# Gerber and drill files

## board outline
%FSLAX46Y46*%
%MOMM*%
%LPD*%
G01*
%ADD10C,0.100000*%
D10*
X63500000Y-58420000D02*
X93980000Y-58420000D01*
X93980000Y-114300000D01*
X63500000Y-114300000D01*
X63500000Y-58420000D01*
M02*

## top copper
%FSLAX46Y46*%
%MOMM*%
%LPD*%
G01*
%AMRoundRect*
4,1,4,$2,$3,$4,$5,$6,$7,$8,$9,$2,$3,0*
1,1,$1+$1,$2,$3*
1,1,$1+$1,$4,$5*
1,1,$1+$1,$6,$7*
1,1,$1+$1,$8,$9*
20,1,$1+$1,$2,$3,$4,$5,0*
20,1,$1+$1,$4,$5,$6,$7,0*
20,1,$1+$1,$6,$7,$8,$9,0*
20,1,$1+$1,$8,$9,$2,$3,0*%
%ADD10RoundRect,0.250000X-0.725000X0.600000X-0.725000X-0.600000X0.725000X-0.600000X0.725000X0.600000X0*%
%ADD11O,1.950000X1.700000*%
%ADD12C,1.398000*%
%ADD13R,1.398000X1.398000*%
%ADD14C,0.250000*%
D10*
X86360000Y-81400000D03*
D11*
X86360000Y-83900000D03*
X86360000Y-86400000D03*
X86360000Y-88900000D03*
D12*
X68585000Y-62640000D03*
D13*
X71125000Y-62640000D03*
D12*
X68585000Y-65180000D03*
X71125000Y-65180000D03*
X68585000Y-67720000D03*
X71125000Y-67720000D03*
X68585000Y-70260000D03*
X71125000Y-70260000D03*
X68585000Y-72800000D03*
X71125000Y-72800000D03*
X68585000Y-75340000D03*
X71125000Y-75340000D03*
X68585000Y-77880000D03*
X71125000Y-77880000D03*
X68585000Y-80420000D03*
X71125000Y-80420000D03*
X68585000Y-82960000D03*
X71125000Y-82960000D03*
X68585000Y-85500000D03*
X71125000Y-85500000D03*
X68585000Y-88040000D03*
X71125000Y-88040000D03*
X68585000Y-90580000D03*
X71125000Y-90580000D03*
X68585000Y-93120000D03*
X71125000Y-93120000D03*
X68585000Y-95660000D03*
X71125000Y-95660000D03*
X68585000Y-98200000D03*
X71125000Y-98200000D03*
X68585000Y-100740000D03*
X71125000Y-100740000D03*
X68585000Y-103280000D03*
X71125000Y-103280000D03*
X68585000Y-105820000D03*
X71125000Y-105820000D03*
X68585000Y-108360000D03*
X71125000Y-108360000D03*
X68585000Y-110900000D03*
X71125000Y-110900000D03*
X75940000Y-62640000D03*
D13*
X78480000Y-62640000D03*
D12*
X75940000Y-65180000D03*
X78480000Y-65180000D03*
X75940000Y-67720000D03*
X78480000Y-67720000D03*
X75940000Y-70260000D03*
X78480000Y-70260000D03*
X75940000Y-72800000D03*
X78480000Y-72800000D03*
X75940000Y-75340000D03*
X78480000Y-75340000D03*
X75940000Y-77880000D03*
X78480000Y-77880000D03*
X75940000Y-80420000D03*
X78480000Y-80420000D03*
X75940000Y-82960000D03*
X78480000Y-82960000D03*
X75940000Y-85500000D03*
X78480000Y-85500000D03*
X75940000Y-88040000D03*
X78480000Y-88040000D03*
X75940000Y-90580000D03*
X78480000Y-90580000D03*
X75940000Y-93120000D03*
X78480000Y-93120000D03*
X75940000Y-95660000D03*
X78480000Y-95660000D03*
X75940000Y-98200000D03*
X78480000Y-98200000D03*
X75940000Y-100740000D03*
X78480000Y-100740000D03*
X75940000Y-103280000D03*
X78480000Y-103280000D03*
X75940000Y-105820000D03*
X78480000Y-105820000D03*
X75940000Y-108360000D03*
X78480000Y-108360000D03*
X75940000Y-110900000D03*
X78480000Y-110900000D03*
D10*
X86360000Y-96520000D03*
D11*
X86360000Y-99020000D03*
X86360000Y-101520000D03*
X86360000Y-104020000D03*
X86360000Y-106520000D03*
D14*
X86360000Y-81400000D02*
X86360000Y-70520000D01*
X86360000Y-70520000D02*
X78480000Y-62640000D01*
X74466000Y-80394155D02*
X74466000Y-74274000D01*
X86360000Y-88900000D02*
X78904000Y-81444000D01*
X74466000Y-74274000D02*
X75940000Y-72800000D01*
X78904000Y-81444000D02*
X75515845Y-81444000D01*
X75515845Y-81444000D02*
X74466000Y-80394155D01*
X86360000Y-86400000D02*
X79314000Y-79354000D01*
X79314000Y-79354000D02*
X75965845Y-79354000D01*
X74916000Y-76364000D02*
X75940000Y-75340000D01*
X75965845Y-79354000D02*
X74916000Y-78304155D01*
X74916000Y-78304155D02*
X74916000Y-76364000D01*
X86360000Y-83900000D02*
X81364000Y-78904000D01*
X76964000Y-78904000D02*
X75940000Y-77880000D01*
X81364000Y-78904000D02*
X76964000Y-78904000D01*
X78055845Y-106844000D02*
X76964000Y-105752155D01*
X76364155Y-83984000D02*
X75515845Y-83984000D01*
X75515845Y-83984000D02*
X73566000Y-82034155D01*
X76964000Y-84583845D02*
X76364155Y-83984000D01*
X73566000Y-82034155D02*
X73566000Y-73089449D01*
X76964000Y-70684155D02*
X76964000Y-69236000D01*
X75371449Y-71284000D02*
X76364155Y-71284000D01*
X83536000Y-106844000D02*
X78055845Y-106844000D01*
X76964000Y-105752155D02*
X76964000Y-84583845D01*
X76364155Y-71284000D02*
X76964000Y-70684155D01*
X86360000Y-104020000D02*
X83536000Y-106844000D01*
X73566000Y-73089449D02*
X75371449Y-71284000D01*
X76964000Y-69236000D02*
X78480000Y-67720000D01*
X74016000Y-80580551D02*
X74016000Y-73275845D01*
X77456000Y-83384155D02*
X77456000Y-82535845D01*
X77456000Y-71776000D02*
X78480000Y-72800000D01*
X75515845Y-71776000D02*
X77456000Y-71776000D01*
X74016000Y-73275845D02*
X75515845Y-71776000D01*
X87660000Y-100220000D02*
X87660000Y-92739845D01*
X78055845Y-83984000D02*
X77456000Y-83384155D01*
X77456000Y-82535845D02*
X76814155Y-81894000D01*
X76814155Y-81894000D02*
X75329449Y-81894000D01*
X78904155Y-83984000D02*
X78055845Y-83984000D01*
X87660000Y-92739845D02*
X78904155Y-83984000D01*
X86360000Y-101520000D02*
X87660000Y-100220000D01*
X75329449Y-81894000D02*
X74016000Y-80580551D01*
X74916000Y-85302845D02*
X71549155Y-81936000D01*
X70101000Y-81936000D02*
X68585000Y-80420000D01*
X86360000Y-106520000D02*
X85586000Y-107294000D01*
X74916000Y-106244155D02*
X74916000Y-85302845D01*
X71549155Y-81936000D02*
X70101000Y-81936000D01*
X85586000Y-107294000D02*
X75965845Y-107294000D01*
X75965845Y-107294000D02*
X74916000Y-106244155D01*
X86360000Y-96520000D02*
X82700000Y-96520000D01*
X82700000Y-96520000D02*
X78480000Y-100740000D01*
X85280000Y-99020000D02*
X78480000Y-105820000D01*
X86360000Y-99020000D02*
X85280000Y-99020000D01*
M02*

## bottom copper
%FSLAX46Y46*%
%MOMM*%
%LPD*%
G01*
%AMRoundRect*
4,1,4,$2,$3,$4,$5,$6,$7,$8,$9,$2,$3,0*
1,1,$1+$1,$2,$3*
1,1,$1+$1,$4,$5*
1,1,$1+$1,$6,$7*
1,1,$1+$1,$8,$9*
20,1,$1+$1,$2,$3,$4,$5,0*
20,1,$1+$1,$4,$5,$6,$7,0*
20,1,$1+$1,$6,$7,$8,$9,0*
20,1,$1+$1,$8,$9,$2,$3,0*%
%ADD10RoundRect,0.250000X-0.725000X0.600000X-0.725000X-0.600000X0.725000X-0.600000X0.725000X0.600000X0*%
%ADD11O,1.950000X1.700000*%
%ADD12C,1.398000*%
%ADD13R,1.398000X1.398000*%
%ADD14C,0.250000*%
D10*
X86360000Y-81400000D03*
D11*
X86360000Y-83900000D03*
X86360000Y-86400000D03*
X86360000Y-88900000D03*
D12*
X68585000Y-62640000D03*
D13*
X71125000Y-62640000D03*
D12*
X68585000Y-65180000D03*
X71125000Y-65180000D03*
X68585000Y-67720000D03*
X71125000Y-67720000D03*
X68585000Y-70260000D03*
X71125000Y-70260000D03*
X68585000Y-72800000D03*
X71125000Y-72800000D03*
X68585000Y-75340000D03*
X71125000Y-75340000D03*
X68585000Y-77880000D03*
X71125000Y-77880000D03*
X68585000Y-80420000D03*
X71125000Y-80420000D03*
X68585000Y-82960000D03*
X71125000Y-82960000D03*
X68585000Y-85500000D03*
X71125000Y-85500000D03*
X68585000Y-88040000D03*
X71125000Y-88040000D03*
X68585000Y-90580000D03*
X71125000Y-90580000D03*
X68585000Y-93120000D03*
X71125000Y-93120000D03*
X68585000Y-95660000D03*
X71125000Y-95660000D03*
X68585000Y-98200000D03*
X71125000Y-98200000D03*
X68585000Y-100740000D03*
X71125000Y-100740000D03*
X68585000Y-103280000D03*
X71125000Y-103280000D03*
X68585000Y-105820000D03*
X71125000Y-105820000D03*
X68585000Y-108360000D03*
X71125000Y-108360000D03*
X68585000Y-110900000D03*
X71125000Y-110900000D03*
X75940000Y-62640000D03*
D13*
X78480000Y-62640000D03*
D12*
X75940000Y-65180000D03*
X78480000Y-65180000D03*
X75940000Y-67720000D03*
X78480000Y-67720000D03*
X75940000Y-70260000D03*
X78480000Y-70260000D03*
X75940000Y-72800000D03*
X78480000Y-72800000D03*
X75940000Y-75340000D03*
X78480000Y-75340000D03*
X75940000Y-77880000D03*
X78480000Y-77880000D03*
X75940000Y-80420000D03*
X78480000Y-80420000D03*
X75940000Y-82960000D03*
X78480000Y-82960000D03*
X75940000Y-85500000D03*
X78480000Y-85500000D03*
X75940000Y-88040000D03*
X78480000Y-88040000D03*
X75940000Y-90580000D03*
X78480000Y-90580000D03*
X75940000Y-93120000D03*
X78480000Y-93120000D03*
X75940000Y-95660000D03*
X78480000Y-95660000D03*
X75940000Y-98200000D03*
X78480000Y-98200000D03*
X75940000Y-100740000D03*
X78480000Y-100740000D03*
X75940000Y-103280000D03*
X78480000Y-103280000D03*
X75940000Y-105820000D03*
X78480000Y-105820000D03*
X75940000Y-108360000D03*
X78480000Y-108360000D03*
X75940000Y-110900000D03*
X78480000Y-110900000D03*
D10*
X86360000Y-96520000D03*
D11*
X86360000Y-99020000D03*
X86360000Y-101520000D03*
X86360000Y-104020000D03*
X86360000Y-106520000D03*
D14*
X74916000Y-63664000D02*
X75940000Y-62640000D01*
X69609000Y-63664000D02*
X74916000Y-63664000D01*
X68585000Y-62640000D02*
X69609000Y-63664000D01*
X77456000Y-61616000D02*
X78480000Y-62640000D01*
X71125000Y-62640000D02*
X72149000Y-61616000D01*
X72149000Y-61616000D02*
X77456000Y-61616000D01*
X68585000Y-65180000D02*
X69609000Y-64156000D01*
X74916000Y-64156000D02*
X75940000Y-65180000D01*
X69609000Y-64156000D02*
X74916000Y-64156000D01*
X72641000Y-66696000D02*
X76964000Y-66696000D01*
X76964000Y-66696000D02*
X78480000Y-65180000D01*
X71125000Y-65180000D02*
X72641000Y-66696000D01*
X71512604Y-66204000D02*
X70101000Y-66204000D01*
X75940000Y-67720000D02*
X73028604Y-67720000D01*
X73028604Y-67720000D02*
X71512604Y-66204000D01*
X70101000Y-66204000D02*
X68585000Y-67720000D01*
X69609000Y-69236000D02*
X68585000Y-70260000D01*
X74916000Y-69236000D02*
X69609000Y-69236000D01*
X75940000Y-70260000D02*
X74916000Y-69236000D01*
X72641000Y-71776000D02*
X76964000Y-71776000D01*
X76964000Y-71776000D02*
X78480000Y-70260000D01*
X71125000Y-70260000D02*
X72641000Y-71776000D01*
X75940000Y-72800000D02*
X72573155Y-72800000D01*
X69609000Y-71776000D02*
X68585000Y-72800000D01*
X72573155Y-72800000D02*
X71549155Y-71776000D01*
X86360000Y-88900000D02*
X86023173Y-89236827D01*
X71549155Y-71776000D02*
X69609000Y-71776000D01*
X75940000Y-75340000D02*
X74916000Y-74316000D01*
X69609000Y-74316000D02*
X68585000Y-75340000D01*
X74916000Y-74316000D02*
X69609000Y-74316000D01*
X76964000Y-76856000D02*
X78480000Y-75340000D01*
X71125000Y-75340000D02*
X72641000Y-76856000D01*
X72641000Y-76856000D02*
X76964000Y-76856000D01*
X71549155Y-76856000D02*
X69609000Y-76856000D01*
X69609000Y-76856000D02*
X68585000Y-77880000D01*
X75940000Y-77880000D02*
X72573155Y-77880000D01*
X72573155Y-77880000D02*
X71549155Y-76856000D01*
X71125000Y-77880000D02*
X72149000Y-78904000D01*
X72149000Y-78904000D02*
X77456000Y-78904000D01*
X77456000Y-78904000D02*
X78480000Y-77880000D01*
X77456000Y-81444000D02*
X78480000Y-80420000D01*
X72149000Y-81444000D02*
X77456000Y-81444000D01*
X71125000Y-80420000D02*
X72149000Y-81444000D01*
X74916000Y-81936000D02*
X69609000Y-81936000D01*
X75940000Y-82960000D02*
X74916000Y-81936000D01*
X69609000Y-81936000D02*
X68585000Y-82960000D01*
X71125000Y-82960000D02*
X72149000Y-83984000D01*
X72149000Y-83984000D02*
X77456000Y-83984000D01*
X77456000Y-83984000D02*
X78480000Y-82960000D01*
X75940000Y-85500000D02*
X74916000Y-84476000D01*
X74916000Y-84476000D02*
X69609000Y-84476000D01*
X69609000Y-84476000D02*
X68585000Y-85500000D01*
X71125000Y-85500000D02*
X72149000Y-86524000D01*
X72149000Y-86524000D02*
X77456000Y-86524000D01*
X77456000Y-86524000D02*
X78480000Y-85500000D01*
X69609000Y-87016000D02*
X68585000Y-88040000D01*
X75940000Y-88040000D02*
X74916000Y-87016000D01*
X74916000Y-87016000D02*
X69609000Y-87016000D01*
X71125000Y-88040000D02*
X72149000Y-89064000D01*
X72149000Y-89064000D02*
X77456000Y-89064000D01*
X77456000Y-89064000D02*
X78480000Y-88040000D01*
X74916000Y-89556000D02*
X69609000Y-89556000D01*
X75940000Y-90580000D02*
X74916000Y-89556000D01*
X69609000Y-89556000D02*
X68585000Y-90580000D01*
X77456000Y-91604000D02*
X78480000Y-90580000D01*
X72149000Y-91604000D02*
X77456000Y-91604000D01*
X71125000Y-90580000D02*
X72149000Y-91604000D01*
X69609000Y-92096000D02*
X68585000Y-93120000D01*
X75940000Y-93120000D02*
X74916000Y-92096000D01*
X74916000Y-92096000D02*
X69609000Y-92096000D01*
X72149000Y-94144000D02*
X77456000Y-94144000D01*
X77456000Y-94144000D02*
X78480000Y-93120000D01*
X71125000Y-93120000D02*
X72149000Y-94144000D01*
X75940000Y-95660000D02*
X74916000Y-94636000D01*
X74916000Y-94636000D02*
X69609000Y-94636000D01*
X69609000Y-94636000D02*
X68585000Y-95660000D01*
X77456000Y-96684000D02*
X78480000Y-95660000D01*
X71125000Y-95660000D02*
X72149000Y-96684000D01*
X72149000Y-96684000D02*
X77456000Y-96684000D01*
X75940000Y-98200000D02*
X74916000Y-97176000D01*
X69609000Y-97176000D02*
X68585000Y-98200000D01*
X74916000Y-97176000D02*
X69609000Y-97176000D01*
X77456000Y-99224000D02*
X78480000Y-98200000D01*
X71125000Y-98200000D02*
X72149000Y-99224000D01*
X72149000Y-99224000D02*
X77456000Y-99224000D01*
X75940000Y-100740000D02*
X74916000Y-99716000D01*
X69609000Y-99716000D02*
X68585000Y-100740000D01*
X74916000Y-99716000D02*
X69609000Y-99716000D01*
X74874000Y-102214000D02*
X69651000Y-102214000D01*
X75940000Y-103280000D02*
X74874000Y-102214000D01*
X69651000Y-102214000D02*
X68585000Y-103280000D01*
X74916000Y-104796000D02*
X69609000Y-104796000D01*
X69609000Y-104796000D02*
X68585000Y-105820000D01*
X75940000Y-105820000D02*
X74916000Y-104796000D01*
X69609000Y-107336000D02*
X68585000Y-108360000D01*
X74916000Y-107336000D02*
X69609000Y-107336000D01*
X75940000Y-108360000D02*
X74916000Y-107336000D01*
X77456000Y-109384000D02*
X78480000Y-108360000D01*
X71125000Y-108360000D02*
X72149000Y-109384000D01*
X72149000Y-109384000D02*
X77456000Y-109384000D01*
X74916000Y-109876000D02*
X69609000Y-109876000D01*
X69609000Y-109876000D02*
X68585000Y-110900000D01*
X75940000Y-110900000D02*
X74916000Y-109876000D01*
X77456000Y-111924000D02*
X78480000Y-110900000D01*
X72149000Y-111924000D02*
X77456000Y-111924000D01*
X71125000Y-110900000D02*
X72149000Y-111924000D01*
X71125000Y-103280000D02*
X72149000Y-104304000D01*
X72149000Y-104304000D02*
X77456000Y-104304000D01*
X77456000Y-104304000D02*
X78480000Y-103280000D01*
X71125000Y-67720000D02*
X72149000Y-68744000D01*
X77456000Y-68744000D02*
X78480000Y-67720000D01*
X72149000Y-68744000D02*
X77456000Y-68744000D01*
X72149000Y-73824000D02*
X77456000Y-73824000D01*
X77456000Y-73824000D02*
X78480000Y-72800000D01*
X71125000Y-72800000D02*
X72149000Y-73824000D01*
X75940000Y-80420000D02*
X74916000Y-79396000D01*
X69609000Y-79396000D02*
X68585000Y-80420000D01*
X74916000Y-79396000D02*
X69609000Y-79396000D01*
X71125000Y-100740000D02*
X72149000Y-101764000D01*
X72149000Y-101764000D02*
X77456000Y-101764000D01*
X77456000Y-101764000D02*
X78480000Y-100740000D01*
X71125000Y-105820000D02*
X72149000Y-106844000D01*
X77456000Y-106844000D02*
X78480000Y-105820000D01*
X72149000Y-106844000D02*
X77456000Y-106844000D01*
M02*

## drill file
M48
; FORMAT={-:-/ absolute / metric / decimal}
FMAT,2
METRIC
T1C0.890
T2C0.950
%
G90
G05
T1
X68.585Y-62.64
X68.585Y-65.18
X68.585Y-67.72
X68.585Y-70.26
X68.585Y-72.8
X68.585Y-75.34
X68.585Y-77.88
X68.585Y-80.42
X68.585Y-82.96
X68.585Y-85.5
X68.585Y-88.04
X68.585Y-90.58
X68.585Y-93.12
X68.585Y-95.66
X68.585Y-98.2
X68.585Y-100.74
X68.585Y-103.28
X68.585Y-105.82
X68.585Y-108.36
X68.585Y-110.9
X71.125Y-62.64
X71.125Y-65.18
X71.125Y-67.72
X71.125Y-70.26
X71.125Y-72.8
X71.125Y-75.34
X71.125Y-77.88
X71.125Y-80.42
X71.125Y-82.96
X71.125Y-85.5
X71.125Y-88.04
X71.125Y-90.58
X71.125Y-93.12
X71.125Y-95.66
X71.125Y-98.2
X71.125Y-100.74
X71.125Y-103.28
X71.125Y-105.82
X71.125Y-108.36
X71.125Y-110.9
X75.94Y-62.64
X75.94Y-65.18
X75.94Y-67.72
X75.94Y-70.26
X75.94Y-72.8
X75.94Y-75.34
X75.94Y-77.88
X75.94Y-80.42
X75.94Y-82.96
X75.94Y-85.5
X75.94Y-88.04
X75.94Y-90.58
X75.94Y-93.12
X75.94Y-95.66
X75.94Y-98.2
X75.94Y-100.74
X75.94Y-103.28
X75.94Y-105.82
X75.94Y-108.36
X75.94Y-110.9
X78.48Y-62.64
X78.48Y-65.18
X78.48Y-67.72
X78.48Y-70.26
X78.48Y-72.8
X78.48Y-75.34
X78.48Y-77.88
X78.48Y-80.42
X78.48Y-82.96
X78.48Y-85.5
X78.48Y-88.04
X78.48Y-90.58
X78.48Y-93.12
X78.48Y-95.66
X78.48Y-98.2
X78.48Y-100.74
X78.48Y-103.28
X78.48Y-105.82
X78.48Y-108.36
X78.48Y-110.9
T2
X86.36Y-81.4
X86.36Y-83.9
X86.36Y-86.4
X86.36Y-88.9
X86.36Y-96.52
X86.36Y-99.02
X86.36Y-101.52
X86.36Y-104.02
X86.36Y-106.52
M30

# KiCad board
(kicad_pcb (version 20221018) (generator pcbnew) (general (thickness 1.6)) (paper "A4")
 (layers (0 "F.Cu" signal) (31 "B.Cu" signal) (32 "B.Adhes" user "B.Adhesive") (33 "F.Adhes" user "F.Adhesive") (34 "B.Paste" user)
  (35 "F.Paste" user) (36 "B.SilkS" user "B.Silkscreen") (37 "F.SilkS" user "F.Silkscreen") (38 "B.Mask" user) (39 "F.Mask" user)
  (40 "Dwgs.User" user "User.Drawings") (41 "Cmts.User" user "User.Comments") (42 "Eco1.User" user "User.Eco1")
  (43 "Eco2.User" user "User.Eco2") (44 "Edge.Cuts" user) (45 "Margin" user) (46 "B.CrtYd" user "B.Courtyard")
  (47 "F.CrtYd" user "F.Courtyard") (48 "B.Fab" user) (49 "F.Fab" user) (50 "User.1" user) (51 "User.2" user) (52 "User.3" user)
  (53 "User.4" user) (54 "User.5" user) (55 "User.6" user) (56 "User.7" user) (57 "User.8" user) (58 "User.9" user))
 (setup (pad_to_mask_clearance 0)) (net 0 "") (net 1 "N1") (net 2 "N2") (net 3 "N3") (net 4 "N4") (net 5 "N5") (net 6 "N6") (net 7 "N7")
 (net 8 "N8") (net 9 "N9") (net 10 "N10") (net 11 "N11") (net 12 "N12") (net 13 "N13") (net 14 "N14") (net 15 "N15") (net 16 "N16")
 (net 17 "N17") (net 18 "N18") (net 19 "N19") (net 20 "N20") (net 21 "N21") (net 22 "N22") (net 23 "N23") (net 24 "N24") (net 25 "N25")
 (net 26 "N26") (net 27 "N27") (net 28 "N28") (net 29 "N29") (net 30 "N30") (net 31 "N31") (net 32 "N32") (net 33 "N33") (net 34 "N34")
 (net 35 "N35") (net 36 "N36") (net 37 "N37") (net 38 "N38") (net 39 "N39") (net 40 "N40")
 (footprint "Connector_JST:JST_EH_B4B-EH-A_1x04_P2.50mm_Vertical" (layer "F.Cu") (at 86.36 81.4 -90)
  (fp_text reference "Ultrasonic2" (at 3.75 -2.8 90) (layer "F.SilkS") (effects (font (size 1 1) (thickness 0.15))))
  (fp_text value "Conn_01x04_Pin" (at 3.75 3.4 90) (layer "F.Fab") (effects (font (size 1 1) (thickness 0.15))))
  (pad "1" thru_hole roundrect (at 0 0 270) (size 1.7 1.95) (drill 0.95) (layers "*.Cu" "*.Mask") (roundrect_rratio 0.1470588235)
   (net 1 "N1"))
  (pad "2" thru_hole oval (at 2.5 0 270) (size 1.7 1.95) (drill 0.95) (layers "*.Cu" "*.Mask") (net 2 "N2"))
  (pad "3" thru_hole oval (at 5 0 270) (size 1.7 1.95) (drill 0.95) (layers "*.Cu" "*.Mask") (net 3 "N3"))
  (pad "4" thru_hole oval (at 7.5 0 270) (size 1.7 1.95) (drill 0.95) (layers "*.Cu" "*.Mask") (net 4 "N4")))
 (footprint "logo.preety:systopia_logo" (layer "F.Cu") (at 87.63 68.58)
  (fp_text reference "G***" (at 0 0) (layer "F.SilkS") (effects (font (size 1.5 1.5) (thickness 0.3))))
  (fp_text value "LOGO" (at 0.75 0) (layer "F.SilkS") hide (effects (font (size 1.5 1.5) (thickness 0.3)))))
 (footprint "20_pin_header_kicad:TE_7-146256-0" (layer "F.Cu") (at 69.855 86.77 -90)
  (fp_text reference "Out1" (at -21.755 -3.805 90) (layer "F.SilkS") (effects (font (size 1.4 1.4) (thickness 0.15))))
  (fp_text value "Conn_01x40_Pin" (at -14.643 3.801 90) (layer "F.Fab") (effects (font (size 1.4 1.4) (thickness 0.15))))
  (pad "1" thru_hole circle (at -24.13 1.27 270) (size 1.398 1.398) (drill 0.89) (layers "*.Cu" "*.Mask") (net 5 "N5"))
  (pad "2" thru_hole rect (at -24.13 -1.27 270) (size 1.398 1.398) (drill 0.89) (layers "*.Cu" "*.Mask") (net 1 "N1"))
  (pad "3" thru_hole circle (at -21.59 1.27 270) (size 1.398 1.398) (drill 0.89) (layers "*.Cu" "*.Mask") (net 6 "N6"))
  (pad "4" thru_hole circle (at -21.59 -1.27 270) (size 1.398 1.398) (drill 0.89) (layers "*.Cu" "*.Mask") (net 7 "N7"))
  (pad "5" thru_hole circle (at -19.05 1.27 270) (size 1.398 1.398) (drill 0.89) (layers "*.Cu" "*.Mask") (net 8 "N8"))
  (pad "6" thru_hole circle (at -19.05 -1.27 270) (size 1.398 1.398) (drill 0.89) (layers "*.Cu" "*.Mask") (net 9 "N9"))
  (pad "7" thru_hole circle (at -16.51 1.27 270) (size 1.398 1.398) (drill 0.89) (layers "*.Cu" "*.Mask") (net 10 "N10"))
  (pad "8" thru_hole circle (at -16.51 -1.27 270) (size 1.398 1.398) (drill 0.89) (layers "*.Cu" "*.Mask") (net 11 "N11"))
  (pad "9" thru_hole circle (at -13.97 1.27 270) (size 1.398 1.398) (drill 0.89) (layers "*.Cu" "*.Mask") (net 4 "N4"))
  (pad "10" thru_hole circle (at -13.97 -1.27 270) (size 1.398 1.398) (drill 0.89) (layers "*.Cu" "*.Mask") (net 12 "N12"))
  (pad "11" thru_hole circle (at -11.43 1.27 270) (size 1.398 1.398) (drill 0.89) (layers "*.Cu" "*.Mask") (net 3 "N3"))
  (pad "12" thru_hole circle (at -11.43 -1.27 270) (size 1.398 1.398) (drill 0.89) (layers "*.Cu" "*.Mask") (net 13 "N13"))
  (pad "13" thru_hole circle (at -8.89 1.27 270) (size 1.398 1.398) (drill 0.89) (layers "*.Cu" "*.Mask") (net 2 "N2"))
  (pad "14" thru_hole circle (at -8.89 -1.27 270) (size 1.398 1.398) (drill 0.89) (layers "*.Cu" "*.Mask") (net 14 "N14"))
  (pad "15" thru_hole circle (at -6.35 1.27 270) (size 1.398 1.398) (drill 0.89) (layers "*.Cu" "*.Mask") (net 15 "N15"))
  (pad "16" thru_hole circle (at -6.35 -1.27 270) (size 1.398 1.398) (drill 0.89) (layers "*.Cu" "*.Mask") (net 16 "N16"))
  (pad "17" thru_hole circle (at -3.81 1.27 270) (size 1.398 1.398) (drill 0.89) (layers "*.Cu" "*.Mask") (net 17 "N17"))
  (pad "18" thru_hole circle (at -3.81 -1.27 270) (size 1.398 1.398) (drill 0.89) (layers "*.Cu" "*.Mask") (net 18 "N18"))
  (pad "19" thru_hole circle (at -1.27 1.27 270) (size 1.398 1.398) (drill 0.89) (layers "*.Cu" "*.Mask") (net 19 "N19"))
  (pad "20" thru_hole circle (at -1.27 -1.27 270) (size 1.398 1.398) (drill 0.89) (layers "*.Cu" "*.Mask") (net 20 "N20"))
  (pad "21" thru_hole circle (at 1.27 1.27 270) (size 1.398 1.398) (drill 0.89) (layers "*.Cu" "*.Mask") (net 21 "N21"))
  (pad "22" thru_hole circle (at 1.27 -1.27 270) (size 1.398 1.398) (drill 0.89) (layers "*.Cu" "*.Mask") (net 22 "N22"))
  (pad "23" thru_hole circle (at 3.81 1.27 270) (size 1.398 1.398) (drill 0.89) (layers "*.Cu" "*.Mask") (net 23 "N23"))
  (pad "24" thru_hole circle (at 3.81 -1.27 270) (size 1.398 1.398) (drill 0.89) (layers "*.Cu" "*.Mask") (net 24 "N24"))
  (pad "25" thru_hole circle (at 6.35 1.27 270) (size 1.398 1.398) (drill 0.89) (layers "*.Cu" "*.Mask") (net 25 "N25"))
  (pad "26" thru_hole circle (at 6.35 -1.27 270) (size 1.398 1.398) (drill 0.89) (layers "*.Cu" "*.Mask") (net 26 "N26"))
  (pad "27" thru_hole circle (at 8.89 1.27 270) (size 1.398 1.398) (drill 0.89) (layers "*.Cu" "*.Mask") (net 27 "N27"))
  (pad "28" thru_hole circle (at 8.89 -1.27 270) (size 1.398 1.398) (drill 0.89) (layers "*.Cu" "*.Mask") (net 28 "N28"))
  (pad "29" thru_hole circle (at 11.43 1.27 270) (size 1.398 1.398) (drill 0.89) (layers "*.Cu" "*.Mask") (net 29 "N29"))
  (pad "30" thru_hole circle (at 11.43 -1.27 270) (size 1.398 1.398) (drill 0.89) (layers "*.Cu" "*.Mask") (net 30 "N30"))
  (pad "31" thru_hole circle (at 13.97 1.27 270) (size 1.398 1.398) (drill 0.89) (layers "*.Cu" "*.Mask") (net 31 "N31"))
  (pad "32" thru_hole circle (at 13.97 -1.27 270) (size 1.398 1.398) (drill 0.89) (layers "*.Cu" "*.Mask") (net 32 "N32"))
  (pad "33" thru_hole circle (at 16.51 1.27 270) (size 1.398 1.398) (drill 0.89) (layers "*.Cu" "*.Mask") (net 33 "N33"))
  (pad "34" thru_hole circle (at 16.51 -1.27 270) (size 1.398 1.398) (drill 0.89) (layers "*.Cu" "*.Mask") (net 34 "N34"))
  (pad "35" thru_hole circle (at 19.05 1.27 270) (size 1.398 1.398) (drill 0.89) (layers "*.Cu" "*.Mask") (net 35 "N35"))
  (pad "36" thru_hole circle (at 19.05 -1.27 270) (size 1.398 1.398) (drill 0.89) (layers "*.Cu" "*.Mask") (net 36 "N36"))
  (pad "37" thru_hole circle (at 21.59 1.27 270) (size 1.398 1.398) (drill 0.89) (layers "*.Cu" "*.Mask") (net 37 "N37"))
  (pad "38" thru_hole circle (at 21.59 -1.27 270) (size 1.398 1.398) (drill 0.89) (layers "*.Cu" "*.Mask") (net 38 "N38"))
  (pad "39" thru_hole circle (at 24.13 1.27 270) (size 1.398 1.398) (drill 0.89) (layers "*.Cu" "*.Mask") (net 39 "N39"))
  (pad "40" thru_hole circle (at 24.13 -1.27 270) (size 1.398 1.398) (drill 0.89) (layers "*.Cu" "*.Mask") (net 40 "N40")))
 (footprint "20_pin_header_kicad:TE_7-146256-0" (layer "F.Cu") (at 77.21 86.77 -90)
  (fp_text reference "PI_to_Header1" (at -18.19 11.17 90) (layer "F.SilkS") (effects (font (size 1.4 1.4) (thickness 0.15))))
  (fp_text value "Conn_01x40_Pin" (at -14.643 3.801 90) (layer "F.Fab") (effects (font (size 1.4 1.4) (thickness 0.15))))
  (pad "1" thru_hole circle (at -24.13 1.27 270) (size 1.398 1.398) (drill 0.89) (layers "*.Cu" "*.Mask") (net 5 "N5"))
  (pad "2" thru_hole rect (at -24.13 -1.27 270) (size 1.398 1.398) (drill 0.89) (layers "*.Cu" "*.Mask") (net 1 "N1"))
  (pad "3" thru_hole circle (at -21.59 1.27 270) (size 1.398 1.398) (drill 0.89) (layers "*.Cu" "*.Mask") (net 6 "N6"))
  (pad "4" thru_hole circle (at -21.59 -1.27 270) (size 1.398 1.398) (drill 0.89) (layers "*.Cu" "*.Mask") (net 7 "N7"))
  (pad "5" thru_hole circle (at -19.05 1.27 270) (size 1.398 1.398) (drill 0.89) (layers "*.Cu" "*.Mask") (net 8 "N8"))
  (pad "6" thru_hole circle (at -19.05 -1.27 270) (size 1.398 1.398) (drill 0.89) (layers "*.Cu" "*.Mask") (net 9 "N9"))
  (pad "7" thru_hole circle (at -16.51 1.27 270) (size 1.398 1.398) (drill 0.89) (layers "*.Cu" "*.Mask") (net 10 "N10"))
  (pad "8" thru_hole circle (at -16.51 -1.27 270) (size 1.398 1.398) (drill 0.89) (layers "*.Cu" "*.Mask") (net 11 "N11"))
  (pad "9" thru_hole circle (at -13.97 1.27 270) (size 1.398 1.398) (drill 0.89) (layers "*.Cu" "*.Mask") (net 4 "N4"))
  (pad "10" thru_hole circle (at -13.97 -1.27 270) (size 1.398 1.398) (drill 0.89) (layers "*.Cu" "*.Mask") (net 12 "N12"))
  (pad "11" thru_hole circle (at -11.43 1.27 270) (size 1.398 1.398) (drill 0.89) (layers "*.Cu" "*.Mask") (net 3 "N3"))
  (pad "12" thru_hole circle (at -11.43 -1.27 270) (size 1.398 1.398) (drill 0.89) (layers "*.Cu" "*.Mask") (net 13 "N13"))
  (pad "13" thru_hole circle (at -8.89 1.27 270) (size 1.398 1.398) (drill 0.89) (layers "*.Cu" "*.Mask") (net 2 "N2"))
  (pad "14" thru_hole circle (at -8.89 -1.27 270) (size 1.398 1.398) (drill 0.89) (layers "*.Cu" "*.Mask") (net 14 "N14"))
  (pad "15" thru_hole circle (at -6.35 1.27 270) (size 1.398 1.398) (drill 0.89) (layers "*.Cu" "*.Mask") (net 15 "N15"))
  (pad "16" thru_hole circle (at -6.35 -1.27 270) (size 1.398 1.398) (drill 0.89) (layers "*.Cu" "*.Mask") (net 16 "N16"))
  (pad "17" thru_hole circle (at -3.81 1.27 270) (size 1.398 1.398) (drill 0.89) (layers "*.Cu" "*.Mask") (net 17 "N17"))
  (pad "18" thru_hole circle (at -3.81 -1.27 270) (size 1.398 1.398) (drill 0.89) (layers "*.Cu" "*.Mask") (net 18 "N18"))
  (pad "19" thru_hole circle (at -1.27 1.27 270) (size 1.398 1.398) (drill 0.89) (layers "*.Cu" "*.Mask") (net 19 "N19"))
  (pad "20" thru_hole circle (at -1.27 -1.27 270) (size 1.398 1.398) (drill 0.89) (layers "*.Cu" "*.Mask") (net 20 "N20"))
  (pad "21" thru_hole circle (at 1.27 1.27 270) (size 1.398 1.398) (drill 0.89) (layers "*.Cu" "*.Mask") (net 21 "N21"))
  (pad "22" thru_hole circle (at 1.27 -1.27 270) (size 1.398 1.398) (drill 0.89) (layers "*.Cu" "*.Mask") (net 22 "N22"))
  (pad "23" thru_hole circle (at 3.81 1.27 270) (size 1.398 1.398) (drill 0.89) (layers "*.Cu" "*.Mask") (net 23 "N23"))
  (pad "24" thru_hole circle (at 3.81 -1.27 270) (size 1.398 1.398) (drill 0.89) (layers "*.Cu" "*.Mask") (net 24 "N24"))
  (pad "25" thru_hole circle (at 6.35 1.27 270) (size 1.398 1.398) (drill 0.89) (layers "*.Cu" "*.Mask") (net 25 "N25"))
  (pad "26" thru_hole circle (at 6.35 -1.27 270) (size 1.398 1.398) (drill 0.89) (layers "*.Cu" "*.Mask") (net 26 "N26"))
  (pad "27" thru_hole circle (at 8.89 1.27 270) (size 1.398 1.398) (drill 0.89) (layers "*.Cu" "*.Mask") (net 27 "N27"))
  (pad "28" thru_hole circle (at 8.89 -1.27 270) (size 1.398 1.398) (drill 0.89) (layers "*.Cu" "*.Mask") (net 28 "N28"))
  (pad "29" thru_hole circle (at 11.43 1.27 270) (size 1.398 1.398) (drill 0.89) (layers "*.Cu" "*.Mask") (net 29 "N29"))
  (pad "30" thru_hole circle (at 11.43 -1.27 270) (size 1.398 1.398) (drill 0.89) (layers "*.Cu" "*.Mask") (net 30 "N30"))
  (pad "31" thru_hole circle (at 13.97 1.27 270) (size 1.398 1.398) (drill 0.89) (layers "*.Cu" "*.Mask") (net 31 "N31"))
  (pad "32" thru_hole circle (at 13.97 -1.27 270) (size 1.398 1.398) (drill 0.89) (layers "*.Cu" "*.Mask") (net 32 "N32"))
  (pad "33" thru_hole circle (at 16.51 1.27 270) (size 1.398 1.398) (drill 0.89) (layers "*.Cu" "*.Mask") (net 33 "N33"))
  (pad "34" thru_hole circle (at 16.51 -1.27 270) (size 1.398 1.398) (drill 0.89) (layers "*.Cu" "*.Mask") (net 34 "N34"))
  (pad "35" thru_hole circle (at 19.05 1.27 270) (size 1.398 1.398) (drill 0.89) (layers "*.Cu" "*.Mask") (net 35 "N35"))
  (pad "36" thru_hole circle (at 19.05 -1.27 270) (size 1.398 1.398) (drill 0.89) (layers "*.Cu" "*.Mask") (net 36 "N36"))
  (pad "37" thru_hole circle (at 21.59 1.27 270) (size 1.398 1.398) (drill 0.89) (layers "*.Cu" "*.Mask") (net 37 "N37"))
  (pad "38" thru_hole circle (at 21.59 -1.27 270) (size 1.398 1.398) (drill 0.89) (layers "*.Cu" "*.Mask") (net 38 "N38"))
  (pad "39" thru_hole circle (at 24.13 1.27 270) (size 1.398 1.398) (drill 0.89) (layers "*.Cu" "*.Mask") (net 39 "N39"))
  (pad "40" thru_hole circle (at 24.13 -1.27 270) (size 1.398 1.398) (drill 0.89) (layers "*.Cu" "*.Mask") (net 40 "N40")))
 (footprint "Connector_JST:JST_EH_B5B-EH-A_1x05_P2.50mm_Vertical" (layer "F.Cu") (at 86.36 96.52 -90)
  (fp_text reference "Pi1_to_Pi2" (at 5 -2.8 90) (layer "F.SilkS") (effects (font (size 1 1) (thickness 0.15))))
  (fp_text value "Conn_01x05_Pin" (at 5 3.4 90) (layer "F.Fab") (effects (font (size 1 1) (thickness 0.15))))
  (pad "1" thru_hole roundrect (at 0 0 270) (size 1.7 1.95) (drill 0.95) (layers "*.Cu" "*.Mask") (roundrect_rratio 0.147059) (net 32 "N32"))
  (pad "2" thru_hole oval (at 2.5 0 270) (size 1.7 1.95) (drill 0.95) (layers "*.Cu" "*.Mask") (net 36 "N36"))
  (pad "3" thru_hole oval (at 5 0 270) (size 1.7 1.95) (drill 0.95) (layers "*.Cu" "*.Mask") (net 12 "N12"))
  (pad "4" thru_hole oval (at 7.5 0 270) (size 1.7 1.95) (drill 0.95) (layers "*.Cu" "*.Mask") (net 9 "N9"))
  (pad "5" thru_hole oval (at 10 0 270) (size 1.7 1.95) (drill 0.95) (layers "*.Cu" "*.Mask") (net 15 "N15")))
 (gr_rect (start 63.5 58.42) (end 93.98 114.3) (stroke (width 0.1) (type default)) (fill none) (layer "Edge.Cuts"))
 (segment (start 74.916 63.664) (end 75.94 62.64) (width 0.25) (layer "B.Cu") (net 5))
 (segment (start 69.609 63.664) (end 74.916 63.664) (width 0.25) (layer "B.Cu") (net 5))
 (segment (start 68.585 62.64) (end 69.609 63.664) (width 0.25) (layer "B.Cu") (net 5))
 (segment (start 86.36 81.4) (end 86.36 70.52) (width 0.25) (layer "F.Cu") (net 1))
 (segment (start 86.36 70.52) (end 78.48 62.64) (width 0.25) (layer "F.Cu") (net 1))
 (segment (start 77.456 61.616) (end 78.48 62.64) (width 0.25) (layer "B.Cu") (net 1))
 (segment (start 71.125 62.64) (end 72.149 61.616) (width 0.25) (layer "B.Cu") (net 1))
 (segment (start 72.149 61.616) (end 77.456 61.616) (width 0.25) (layer "B.Cu") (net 1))
 (segment (start 68.585 65.18) (end 69.609 64.156) (width 0.25) (layer "B.Cu") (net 6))
 (segment (start 74.916 64.156) (end 75.94 65.18) (width 0.25) (layer "B.Cu") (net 6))
 (segment (start 69.609 64.156) (end 74.916 64.156) (width 0.25) (layer "B.Cu") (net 6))
 (segment (start 72.641 66.696) (end 76.964 66.696) (width 0.25) (layer "B.Cu") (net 7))
 (segment (start 76.964 66.696) (end 78.48 65.18) (width 0.25) (layer "B.Cu") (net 7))
 (segment (start 71.125 65.18) (end 72.641 66.696) (width 0.25) (layer "B.Cu") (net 7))
 (segment (start 71.512604 66.204) (end 70.101 66.204) (width 0.25) (layer "B.Cu") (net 8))
 (segment (start 75.94 67.72) (end 73.028604 67.72) (width 0.25) (layer "B.Cu") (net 8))
 (segment (start 73.028604 67.72) (end 71.512604 66.204) (width 0.25) (layer "B.Cu") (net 8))
 (segment (start 70.101 66.204) (end 68.585 67.72) (width 0.25) (layer "B.Cu") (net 8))
 (segment (start 69.609 69.236) (end 68.585 70.26) (width 0.25) (layer "B.Cu") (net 10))
 (segment (start 74.916 69.236) (end 69.609 69.236) (width 0.25) (layer "B.Cu") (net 10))
 (segment (start 75.94 70.26) (end 74.916 69.236) (width 0.25) (layer "B.Cu") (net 10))
 (segment (start 72.641 71.776) (end 76.964 71.776) (width 0.25) (layer "B.Cu") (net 11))
 (segment (start 76.964 71.776) (end 78.48 70.26) (width 0.25) (layer "B.Cu") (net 11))
 (segment (start 71.125 70.26) (end 72.641 71.776) (width 0.25) (layer "B.Cu") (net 11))
 (segment (start 74.466 80.394155) (end 74.466 74.274) (width 0.25) (layer "F.Cu") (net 4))
 (segment (start 86.36 88.9) (end 78.904 81.444) (width 0.25) (layer "F.Cu") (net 4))
 (segment (start 74.466 74.274) (end 75.94 72.8) (width 0.25) (layer "F.Cu") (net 4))
 (segment (start 78.904 81.444) (end 75.515845 81.444) (width 0.25) (layer "F.Cu") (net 4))
 (segment (start 75.515845 81.444) (end 74.466 80.394155) (width 0.25) (layer "F.Cu") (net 4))
 (segment (start 75.94 72.8) (end 72.573155 72.8) (width 0.25) (layer "B.Cu") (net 4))
 (segment (start 69.609 71.776) (end 68.585 72.8) (width 0.25) (layer "B.Cu") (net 4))
 (segment (start 72.573155 72.8) (end 71.549155 71.776) (width 0.25) (layer "B.Cu") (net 4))
 (segment (start 86.36 88.9) (end 86.023173 89.236827) (width 0.25) (layer "B.Cu") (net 4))
 (segment (start 71.549155 71.776) (end 69.609 71.776) (width 0.25) (layer "B.Cu") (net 4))
 (segment (start 86.36 86.4) (end 79.314 79.354) (width 0.25) (layer "F.Cu") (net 3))
 (segment (start 79.314 79.354) (end 75.965845 79.354) (width 0.25) (layer "F.Cu") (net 3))
 (segment (start 74.916 76.364) (end 75.94 75.34) (width 0.25) (layer "F.Cu") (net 3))
 (segment (start 75.965845 79.354) (end 74.916 78.304155) (width 0.25) (layer "F.Cu") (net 3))
 (segment (start 74.916 78.304155) (end 74.916 76.364) (width 0.25) (layer "F.Cu") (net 3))
 (segment (start 75.94 75.34) (end 74.916 74.316) (width 0.25) (layer "B.Cu") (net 3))
 (segment (start 69.609 74.316) (end 68.585 75.34) (width 0.25) (layer "B.Cu") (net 3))
 (segment (start 74.916 74.316) (end 69.609 74.316) (width 0.25) (layer "B.Cu") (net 3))
 (segment (start 76.964 76.856) (end 78.48 75.34) (width 0.25) (layer "B.Cu") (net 13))
 (segment (start 71.125 75.34) (end 72.641 76.856) (width 0.25) (layer "B.Cu") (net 13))
 (segment (start 72.641 76.856) (end 76.964 76.856) (width 0.25) (layer "B.Cu") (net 13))
 (segment (start 86.36 83.9) (end 81.364 78.904) (width 0.25) (layer "F.Cu") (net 2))
 (segment (start 76.964 78.904) (end 75.94 77.88) (width 0.25) (layer "F.Cu") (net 2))
 (segment (start 81.364 78.904) (end 76.964 78.904) (width 0.25) (layer "F.Cu") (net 2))
 (segment (start 71.549155 76.856) (end 69.609 76.856) (width 0.25) (layer "B.Cu") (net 2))
 (segment (start 69.609 76.856) (end 68.585 77.88) (width 0.25) (layer "B.Cu") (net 2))
 (segment (start 75.94 77.88) (end 72.573155 77.88) (width 0.25) (layer "B.Cu") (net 2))
 (segment (start 72.573155 77.88) (end 71.549155 76.856) (width 0.25) (layer "B.Cu") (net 2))
 (segment (start 71.125 77.88) (end 72.149 78.904) (width 0.25) (layer "B.Cu") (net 14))
 (segment (start 72.149 78.904) (end 77.456 78.904) (width 0.25) (layer "B.Cu") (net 14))
 (segment (start 77.456 78.904) (end 78.48 77.88) (width 0.25) (layer "B.Cu") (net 14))
 (segment (start 77.456 81.444) (end 78.48 80.42) (width 0.25) (layer "B.Cu") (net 16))
 (segment (start 72.149 81.444) (end 77.456 81.444) (width 0.25) (layer "B.Cu") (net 16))
 (segment (start 71.125 80.42) (end 72.149 81.444) (width 0.25) (layer "B.Cu") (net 16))
 (segment (start 74.916 81.936) (end 69.609 81.936) (width 0.25) (layer "B.Cu") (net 17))
 (segment (start 75.94 82.96) (end 74.916 81.936) (width 0.25) (layer "B.Cu") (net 17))
 (segment (start 69.609 81.936) (end 68.585 82.96) (width 0.25) (layer "B.Cu") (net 17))
 (segment (start 71.125 82.96) (end 72.149 83.984) (width 0.25) (layer "B.Cu") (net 18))
 (segment (start 72.149 83.984) (end 77.456 83.984) (width 0.25) (layer "B.Cu") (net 18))
 (segment (start 77.456 83.984) (end 78.48 82.96) (width 0.25) (layer "B.Cu") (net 18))
 (segment (start 75.94 85.5) (end 74.916 84.476) (width 0.25) (layer "B.Cu") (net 19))
 (segment (start 74.916 84.476) (end 69.609 84.476) (width 0.25) (layer "B.Cu") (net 19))
 (segment (start 69.609 84.476) (end 68.585 85.5) (width 0.25) (layer "B.Cu") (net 19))
 (segment (start 71.125 85.5) (end 72.149 86.524) (width 0.25) (layer "B.Cu") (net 20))
 (segment (start 72.149 86.524) (end 77.456 86.524) (width 0.25) (layer "B.Cu") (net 20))
 (segment (start 77.456 86.524) (end 78.48 85.5) (width 0.25) (layer "B.Cu") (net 20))
 (segment (start 69.609 87.016) (end 68.585 88.04) (width 0.25) (layer "B.Cu") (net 21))
 (segment (start 75.94 88.04) (end 74.916 87.016) (width 0.25) (layer "B.Cu") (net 21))
 (segment (start 74.916 87.016) (end 69.609 87.016) (width 0.25) (layer "B.Cu") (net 21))
 (segment (start 71.125 88.04) (end 72.149 89.064) (width 0.25) (layer "B.Cu") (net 22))
 (segment (start 72.149 89.064) (end 77.456 89.064) (width 0.25) (layer "B.Cu") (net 22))
 (segment (start 77.456 89.064) (end 78.48 88.04) (width 0.25) (layer "B.Cu") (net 22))
 (segment (start 74.916 89.556) (end 69.609 89.556) (width 0.25) (layer "B.Cu") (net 23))
 (segment (start 75.94 90.58) (end 74.916 89.556) (width 0.25) (layer "B.Cu") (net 23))
 (segment (start 69.609 89.556) (end 68.585 90.58) (width 0.25) (layer "B.Cu") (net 23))
 (segment (start 77.456 91.604) (end 78.48 90.58) (width 0.25) (layer "B.Cu") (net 24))
 (segment (start 72.149 91.604) (end 77.456 91.604) (width 0.25) (layer "B.Cu") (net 24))
 (segment (start 71.125 90.58) (end 72.149 91.604) (width 0.25) (layer "B.Cu") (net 24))
 (segment (start 69.609 92.096) (end 68.585 93.12) (width 0.25) (layer "B.Cu") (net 25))
 (segment (start 75.94 93.12) (end 74.916 92.096) (width 0.25) (layer "B.Cu") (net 25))
 (segment (start 74.916 92.096) (end 69.609 92.096) (width 0.25) (layer "B.Cu") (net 25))
 (segment (start 72.149 94.144) (end 77.456 94.144) (width 0.25) (layer "B.Cu") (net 26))
 (segment (start 77.456 94.144) (end 78.48 93.12) (width 0.25) (layer "B.Cu") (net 26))
 (segment (start 71.125 93.12) (end 72.149 94.144) (width 0.25) (layer "B.Cu") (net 26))
 (segment (start 75.94 95.66) (end 74.916 94.636) (width 0.25) (layer "B.Cu") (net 27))
 (segment (start 74.916 94.636) (end 69.609 94.636) (width 0.25) (layer "B.Cu") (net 27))
 (segment (start 69.609 94.636) (end 68.585 95.66) (width 0.25) (layer "B.Cu") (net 27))
 (segment (start 77.456 96.684) (end 78.48 95.66) (width 0.25) (layer "B.Cu") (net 28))
 (segment (start 71.125 95.66) (end 72.149 96.684) (width 0.25) (layer "B.Cu") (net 28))
 (segment (start 72.149 96.684) (end 77.456 96.684) (width 0.25) (layer "B.Cu") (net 28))
 (segment (start 75.94 98.2) (end 74.916 97.176) (width 0.25) (layer "B.Cu") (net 29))
 (segment (start 69.609 97.176) (end 68.585 98.2) (width 0.25) (layer "B.Cu") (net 29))
 (segment (start 74.916 97.176) (end 69.609 97.176) (width 0.25) (layer "B.Cu") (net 29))
 (segment (start 77.456 99.224) (end 78.48 98.2) (width 0.25) (layer "B.Cu") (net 30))
 (segment (start 71.125 98.2) (end 72.149 99.224) (width 0.25) (layer "B.Cu") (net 30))
 (segment (start 72.149 99.224) (end 77.456 99.224) (width 0.25) (layer "B.Cu") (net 30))
 (segment (start 75.94 100.74) (end 74.916 99.716) (width 0.25) (layer "B.Cu") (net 31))
 (segment (start 69.609 99.716) (end 68.585 100.74) (width 0.25) (layer "B.Cu") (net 31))
 (segment (start 74.916 99.716) (end 69.609 99.716) (width 0.25) (layer "B.Cu") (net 31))
 (segment (start 74.874 102.214) (end 69.651 102.214) (width 0.25) (layer "B.Cu") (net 33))
 (segment (start 75.94 103.28) (end 74.874 102.214) (width 0.25) (layer "B.Cu") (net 33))
 (segment (start 69.651 102.214) (end 68.585 103.28) (width 0.25) (layer "B.Cu") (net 33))
 (segment (start 74.916 104.796) (end 69.609 104.796) (width 0.25) (layer "B.Cu") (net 35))
 (segment (start 69.609 104.796) (end 68.585 105.82) (width 0.25) (layer "B.Cu") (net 35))
 (segment (start 75.94 105.82) (end 74.916 104.796) (width 0.25) (layer "B.Cu") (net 35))
 (segment (start 69.609 107.336) (end 68.585 108.36) (width 0.25) (layer "B.Cu") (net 37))
 (segment (start 74.916 107.336) (end 69.609 107.336) (width 0.25) (layer "B.Cu") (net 37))
 (segment (start 75.94 108.36) (end 74.916 107.336) (width 0.25) (layer "B.Cu") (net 37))
 (segment (start 77.456 109.384) (end 78.48 108.36) (width 0.25) (layer "B.Cu") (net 38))
 (segment (start 71.125 108.36) (end 72.149 109.384) (width 0.25) (layer "B.Cu") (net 38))
 (segment (start 72.149 109.384) (end 77.456 109.384) (width 0.25) (layer "B.Cu") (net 38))
 (segment (start 74.916 109.876) (end 69.609 109.876) (width 0.25) (layer "B.Cu") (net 39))
 (segment (start 69.609 109.876) (end 68.585 110.9) (width 0.25) (layer "B.Cu") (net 39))
 (segment (start 75.94 110.9) (end 74.916 109.876) (width 0.25) (layer "B.Cu") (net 39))
 (segment (start 77.456 111.924) (end 78.48 110.9) (width 0.25) (layer "B.Cu") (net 40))
 (segment (start 72.149 111.924) (end 77.456 111.924) (width 0.25) (layer "B.Cu") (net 40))
 (segment (start 71.125 110.9) (end 72.149 111.924) (width 0.25) (layer "B.Cu") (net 40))
 (segment (start 71.125 103.28) (end 72.149 104.304) (width 0.25) (layer "B.Cu") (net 34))
 (segment (start 72.149 104.304) (end 77.456 104.304) (width 0.25) (layer "B.Cu") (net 34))
 (segment (start 77.456 104.304) (end 78.48 103.28) (width 0.25) (layer "B.Cu") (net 34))
 (segment (start 78.055845 106.844) (end 76.964 105.752155) (width 0.25) (layer "F.Cu") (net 9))
 (segment (start 76.364155 83.984) (end 75.515845 83.984) (width 0.25) (layer "F.Cu") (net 9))
 (segment (start 75.515845 83.984) (end 73.566 82.034155) (width 0.25) (layer "F.Cu") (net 9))
 (segment (start 76.964 84.583845) (end 76.364155 83.984) (width 0.25) (layer "F.Cu") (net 9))
 (segment (start 73.566 82.034155) (end 73.566 73.089449) (width 0.25) (layer "F.Cu") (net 9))
 (segment (start 76.964 70.684155) (end 76.964 69.236) (width 0.25) (layer "F.Cu") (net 9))
 (segment (start 75.371449 71.284) (end 76.364155 71.284) (width 0.25) (layer "F.Cu") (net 9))
 (segment (start 83.536 106.844) (end 78.055845 106.844) (width 0.25) (layer "F.Cu") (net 9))
 (segment (start 76.964 105.752155) (end 76.964 84.583845) (width 0.25) (layer "F.Cu") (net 9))
 (segment (start 76.364155 71.284) (end 76.964 70.684155) (width 0.25) (layer "F.Cu") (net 9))
 (segment (start 86.36 104.02) (end 83.536 106.844) (width 0.25) (layer "F.Cu") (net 9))
 (segment (start 73.566 73.089449) (end 75.371449 71.284) (width 0.25) (layer "F.Cu") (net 9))
 (segment (start 76.964 69.236) (end 78.48 67.72) (width 0.25) (layer "F.Cu") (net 9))
 (segment (start 71.125 67.72) (end 72.149 68.744) (width 0.25) (layer "B.Cu") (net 9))
 (segment (start 77.456 68.744) (end 78.48 67.72) (width 0.25) (layer "B.Cu") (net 9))
 (segment (start 72.149 68.744) (end 77.456 68.744) (width 0.25) (layer "B.Cu") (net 9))
 (segment (start 74.016 80.580551) (end 74.016 73.275845) (width 0.25) (layer "F.Cu") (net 12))
 (segment (start 77.456 83.384155) (end 77.456 82.535845) (width 0.25) (layer "F.Cu") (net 12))
 (segment (start 77.456 71.776) (end 78.48 72.8) (width 0.25) (layer "F.Cu") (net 12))
 (segment (start 75.515845 71.776) (end 77.456 71.776) (width 0.25) (layer "F.Cu") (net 12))
 (segment (start 74.016 73.275845) (end 75.515845 71.776) (width 0.25) (layer "F.Cu") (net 12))
 (segment (start 87.66 100.22) (end 87.66 92.739845) (width 0.25) (layer "F.Cu") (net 12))
 (segment (start 78.055845 83.984) (end 77.456 83.384155) (width 0.25) (layer "F.Cu") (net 12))
 (segment (start 77.456 82.535845) (end 76.814155 81.894) (width 0.25) (layer "F.Cu") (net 12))
 (segment (start 76.814155 81.894) (end 75.329449 81.894) (width 0.25) (layer "F.Cu") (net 12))
 (segment (start 78.904155 83.984) (end 78.055845 83.984) (width 0.25) (layer "F.Cu") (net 12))
 (segment (start 87.66 92.739845) (end 78.904155 83.984) (width 0.25) (layer "F.Cu") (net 12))
 (segment (start 86.36 101.52) (end 87.66 100.22) (width 0.25) (layer "F.Cu") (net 12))
 (segment (start 75.329449 81.894) (end 74.016 80.580551) (width 0.25) (layer "F.Cu") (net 12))
 (segment (start 72.149 73.824) (end 77.456 73.824) (width 0.25) (layer "B.Cu") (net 12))
 (segment (start 77.456 73.824) (end 78.48 72.8) (width 0.25) (layer "B.Cu") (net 12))
 (segment (start 71.125 72.8) (end 72.149 73.824) (width 0.25) (layer "B.Cu") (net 12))
 (segment (start 74.916 85.302845) (end 71.549155 81.936) (width 0.25) (layer "F.Cu") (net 15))
 (segment (start 70.101 81.936) (end 68.585 80.42) (width 0.25) (layer "F.Cu") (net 15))
 (segment (start 86.36 106.52) (end 85.586 107.294) (width 0.25) (layer "F.Cu") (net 15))
 (segment (start 74.916 106.244155) (end 74.916 85.302845) (width 0.25) (layer "F.Cu") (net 15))
 (segment (start 71.549155 81.936) (end 70.101 81.936) (width 0.25) (layer "F.Cu") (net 15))
 (segment (start 85.586 107.294) (end 75.965845 107.294) (width 0.25) (layer "F.Cu") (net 15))
 (segment (start 75.965845 107.294) (end 74.916 106.244155) (width 0.25) (layer "F.Cu") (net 15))
 (segment (start 75.94 80.42) (end 74.916 79.396) (width 0.25) (layer "B.Cu") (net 15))
 (segment (start 69.609 79.396) (end 68.585 80.42) (width 0.25) (layer "B.Cu") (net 15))
 (segment (start 74.916 79.396) (end 69.609 79.396) (width 0.25) (layer "B.Cu") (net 15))
 (segment (start 86.36 96.52) (end 82.7 96.52) (width 0.25) (layer "F.Cu") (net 32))
 (segment (start 82.7 96.52) (end 78.48 100.74) (width 0.25) (layer "F.Cu") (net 32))
 (segment (start 71.125 100.74) (end 72.149 101.764) (width 0.25) (layer "B.Cu") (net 32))
 (segment (start 72.149 101.764) (end 77.456 101.764) (width 0.25) (layer "B.Cu") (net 32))
 (segment (start 77.456 101.764) (end 78.48 100.74) (width 0.25) (layer "B.Cu") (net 32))
 (segment (start 85.28 99.02) (end 78.48 105.82) (width 0.25) (layer "F.Cu") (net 36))
 (segment (start 86.36 99.02) (end 85.28 99.02) (width 0.25) (layer "F.Cu") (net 36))
 (segment (start 71.125 105.82) (end 72.149 106.844) (width 0.25) (layer "B.Cu") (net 36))
 (segment (start 77.456 106.844) (end 78.48 105.82) (width 0.25) (layer "B.Cu") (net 36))
 (segment (start 72.149 106.844) (end 77.456 106.844) (width 0.25) (layer "B.Cu") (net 36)))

